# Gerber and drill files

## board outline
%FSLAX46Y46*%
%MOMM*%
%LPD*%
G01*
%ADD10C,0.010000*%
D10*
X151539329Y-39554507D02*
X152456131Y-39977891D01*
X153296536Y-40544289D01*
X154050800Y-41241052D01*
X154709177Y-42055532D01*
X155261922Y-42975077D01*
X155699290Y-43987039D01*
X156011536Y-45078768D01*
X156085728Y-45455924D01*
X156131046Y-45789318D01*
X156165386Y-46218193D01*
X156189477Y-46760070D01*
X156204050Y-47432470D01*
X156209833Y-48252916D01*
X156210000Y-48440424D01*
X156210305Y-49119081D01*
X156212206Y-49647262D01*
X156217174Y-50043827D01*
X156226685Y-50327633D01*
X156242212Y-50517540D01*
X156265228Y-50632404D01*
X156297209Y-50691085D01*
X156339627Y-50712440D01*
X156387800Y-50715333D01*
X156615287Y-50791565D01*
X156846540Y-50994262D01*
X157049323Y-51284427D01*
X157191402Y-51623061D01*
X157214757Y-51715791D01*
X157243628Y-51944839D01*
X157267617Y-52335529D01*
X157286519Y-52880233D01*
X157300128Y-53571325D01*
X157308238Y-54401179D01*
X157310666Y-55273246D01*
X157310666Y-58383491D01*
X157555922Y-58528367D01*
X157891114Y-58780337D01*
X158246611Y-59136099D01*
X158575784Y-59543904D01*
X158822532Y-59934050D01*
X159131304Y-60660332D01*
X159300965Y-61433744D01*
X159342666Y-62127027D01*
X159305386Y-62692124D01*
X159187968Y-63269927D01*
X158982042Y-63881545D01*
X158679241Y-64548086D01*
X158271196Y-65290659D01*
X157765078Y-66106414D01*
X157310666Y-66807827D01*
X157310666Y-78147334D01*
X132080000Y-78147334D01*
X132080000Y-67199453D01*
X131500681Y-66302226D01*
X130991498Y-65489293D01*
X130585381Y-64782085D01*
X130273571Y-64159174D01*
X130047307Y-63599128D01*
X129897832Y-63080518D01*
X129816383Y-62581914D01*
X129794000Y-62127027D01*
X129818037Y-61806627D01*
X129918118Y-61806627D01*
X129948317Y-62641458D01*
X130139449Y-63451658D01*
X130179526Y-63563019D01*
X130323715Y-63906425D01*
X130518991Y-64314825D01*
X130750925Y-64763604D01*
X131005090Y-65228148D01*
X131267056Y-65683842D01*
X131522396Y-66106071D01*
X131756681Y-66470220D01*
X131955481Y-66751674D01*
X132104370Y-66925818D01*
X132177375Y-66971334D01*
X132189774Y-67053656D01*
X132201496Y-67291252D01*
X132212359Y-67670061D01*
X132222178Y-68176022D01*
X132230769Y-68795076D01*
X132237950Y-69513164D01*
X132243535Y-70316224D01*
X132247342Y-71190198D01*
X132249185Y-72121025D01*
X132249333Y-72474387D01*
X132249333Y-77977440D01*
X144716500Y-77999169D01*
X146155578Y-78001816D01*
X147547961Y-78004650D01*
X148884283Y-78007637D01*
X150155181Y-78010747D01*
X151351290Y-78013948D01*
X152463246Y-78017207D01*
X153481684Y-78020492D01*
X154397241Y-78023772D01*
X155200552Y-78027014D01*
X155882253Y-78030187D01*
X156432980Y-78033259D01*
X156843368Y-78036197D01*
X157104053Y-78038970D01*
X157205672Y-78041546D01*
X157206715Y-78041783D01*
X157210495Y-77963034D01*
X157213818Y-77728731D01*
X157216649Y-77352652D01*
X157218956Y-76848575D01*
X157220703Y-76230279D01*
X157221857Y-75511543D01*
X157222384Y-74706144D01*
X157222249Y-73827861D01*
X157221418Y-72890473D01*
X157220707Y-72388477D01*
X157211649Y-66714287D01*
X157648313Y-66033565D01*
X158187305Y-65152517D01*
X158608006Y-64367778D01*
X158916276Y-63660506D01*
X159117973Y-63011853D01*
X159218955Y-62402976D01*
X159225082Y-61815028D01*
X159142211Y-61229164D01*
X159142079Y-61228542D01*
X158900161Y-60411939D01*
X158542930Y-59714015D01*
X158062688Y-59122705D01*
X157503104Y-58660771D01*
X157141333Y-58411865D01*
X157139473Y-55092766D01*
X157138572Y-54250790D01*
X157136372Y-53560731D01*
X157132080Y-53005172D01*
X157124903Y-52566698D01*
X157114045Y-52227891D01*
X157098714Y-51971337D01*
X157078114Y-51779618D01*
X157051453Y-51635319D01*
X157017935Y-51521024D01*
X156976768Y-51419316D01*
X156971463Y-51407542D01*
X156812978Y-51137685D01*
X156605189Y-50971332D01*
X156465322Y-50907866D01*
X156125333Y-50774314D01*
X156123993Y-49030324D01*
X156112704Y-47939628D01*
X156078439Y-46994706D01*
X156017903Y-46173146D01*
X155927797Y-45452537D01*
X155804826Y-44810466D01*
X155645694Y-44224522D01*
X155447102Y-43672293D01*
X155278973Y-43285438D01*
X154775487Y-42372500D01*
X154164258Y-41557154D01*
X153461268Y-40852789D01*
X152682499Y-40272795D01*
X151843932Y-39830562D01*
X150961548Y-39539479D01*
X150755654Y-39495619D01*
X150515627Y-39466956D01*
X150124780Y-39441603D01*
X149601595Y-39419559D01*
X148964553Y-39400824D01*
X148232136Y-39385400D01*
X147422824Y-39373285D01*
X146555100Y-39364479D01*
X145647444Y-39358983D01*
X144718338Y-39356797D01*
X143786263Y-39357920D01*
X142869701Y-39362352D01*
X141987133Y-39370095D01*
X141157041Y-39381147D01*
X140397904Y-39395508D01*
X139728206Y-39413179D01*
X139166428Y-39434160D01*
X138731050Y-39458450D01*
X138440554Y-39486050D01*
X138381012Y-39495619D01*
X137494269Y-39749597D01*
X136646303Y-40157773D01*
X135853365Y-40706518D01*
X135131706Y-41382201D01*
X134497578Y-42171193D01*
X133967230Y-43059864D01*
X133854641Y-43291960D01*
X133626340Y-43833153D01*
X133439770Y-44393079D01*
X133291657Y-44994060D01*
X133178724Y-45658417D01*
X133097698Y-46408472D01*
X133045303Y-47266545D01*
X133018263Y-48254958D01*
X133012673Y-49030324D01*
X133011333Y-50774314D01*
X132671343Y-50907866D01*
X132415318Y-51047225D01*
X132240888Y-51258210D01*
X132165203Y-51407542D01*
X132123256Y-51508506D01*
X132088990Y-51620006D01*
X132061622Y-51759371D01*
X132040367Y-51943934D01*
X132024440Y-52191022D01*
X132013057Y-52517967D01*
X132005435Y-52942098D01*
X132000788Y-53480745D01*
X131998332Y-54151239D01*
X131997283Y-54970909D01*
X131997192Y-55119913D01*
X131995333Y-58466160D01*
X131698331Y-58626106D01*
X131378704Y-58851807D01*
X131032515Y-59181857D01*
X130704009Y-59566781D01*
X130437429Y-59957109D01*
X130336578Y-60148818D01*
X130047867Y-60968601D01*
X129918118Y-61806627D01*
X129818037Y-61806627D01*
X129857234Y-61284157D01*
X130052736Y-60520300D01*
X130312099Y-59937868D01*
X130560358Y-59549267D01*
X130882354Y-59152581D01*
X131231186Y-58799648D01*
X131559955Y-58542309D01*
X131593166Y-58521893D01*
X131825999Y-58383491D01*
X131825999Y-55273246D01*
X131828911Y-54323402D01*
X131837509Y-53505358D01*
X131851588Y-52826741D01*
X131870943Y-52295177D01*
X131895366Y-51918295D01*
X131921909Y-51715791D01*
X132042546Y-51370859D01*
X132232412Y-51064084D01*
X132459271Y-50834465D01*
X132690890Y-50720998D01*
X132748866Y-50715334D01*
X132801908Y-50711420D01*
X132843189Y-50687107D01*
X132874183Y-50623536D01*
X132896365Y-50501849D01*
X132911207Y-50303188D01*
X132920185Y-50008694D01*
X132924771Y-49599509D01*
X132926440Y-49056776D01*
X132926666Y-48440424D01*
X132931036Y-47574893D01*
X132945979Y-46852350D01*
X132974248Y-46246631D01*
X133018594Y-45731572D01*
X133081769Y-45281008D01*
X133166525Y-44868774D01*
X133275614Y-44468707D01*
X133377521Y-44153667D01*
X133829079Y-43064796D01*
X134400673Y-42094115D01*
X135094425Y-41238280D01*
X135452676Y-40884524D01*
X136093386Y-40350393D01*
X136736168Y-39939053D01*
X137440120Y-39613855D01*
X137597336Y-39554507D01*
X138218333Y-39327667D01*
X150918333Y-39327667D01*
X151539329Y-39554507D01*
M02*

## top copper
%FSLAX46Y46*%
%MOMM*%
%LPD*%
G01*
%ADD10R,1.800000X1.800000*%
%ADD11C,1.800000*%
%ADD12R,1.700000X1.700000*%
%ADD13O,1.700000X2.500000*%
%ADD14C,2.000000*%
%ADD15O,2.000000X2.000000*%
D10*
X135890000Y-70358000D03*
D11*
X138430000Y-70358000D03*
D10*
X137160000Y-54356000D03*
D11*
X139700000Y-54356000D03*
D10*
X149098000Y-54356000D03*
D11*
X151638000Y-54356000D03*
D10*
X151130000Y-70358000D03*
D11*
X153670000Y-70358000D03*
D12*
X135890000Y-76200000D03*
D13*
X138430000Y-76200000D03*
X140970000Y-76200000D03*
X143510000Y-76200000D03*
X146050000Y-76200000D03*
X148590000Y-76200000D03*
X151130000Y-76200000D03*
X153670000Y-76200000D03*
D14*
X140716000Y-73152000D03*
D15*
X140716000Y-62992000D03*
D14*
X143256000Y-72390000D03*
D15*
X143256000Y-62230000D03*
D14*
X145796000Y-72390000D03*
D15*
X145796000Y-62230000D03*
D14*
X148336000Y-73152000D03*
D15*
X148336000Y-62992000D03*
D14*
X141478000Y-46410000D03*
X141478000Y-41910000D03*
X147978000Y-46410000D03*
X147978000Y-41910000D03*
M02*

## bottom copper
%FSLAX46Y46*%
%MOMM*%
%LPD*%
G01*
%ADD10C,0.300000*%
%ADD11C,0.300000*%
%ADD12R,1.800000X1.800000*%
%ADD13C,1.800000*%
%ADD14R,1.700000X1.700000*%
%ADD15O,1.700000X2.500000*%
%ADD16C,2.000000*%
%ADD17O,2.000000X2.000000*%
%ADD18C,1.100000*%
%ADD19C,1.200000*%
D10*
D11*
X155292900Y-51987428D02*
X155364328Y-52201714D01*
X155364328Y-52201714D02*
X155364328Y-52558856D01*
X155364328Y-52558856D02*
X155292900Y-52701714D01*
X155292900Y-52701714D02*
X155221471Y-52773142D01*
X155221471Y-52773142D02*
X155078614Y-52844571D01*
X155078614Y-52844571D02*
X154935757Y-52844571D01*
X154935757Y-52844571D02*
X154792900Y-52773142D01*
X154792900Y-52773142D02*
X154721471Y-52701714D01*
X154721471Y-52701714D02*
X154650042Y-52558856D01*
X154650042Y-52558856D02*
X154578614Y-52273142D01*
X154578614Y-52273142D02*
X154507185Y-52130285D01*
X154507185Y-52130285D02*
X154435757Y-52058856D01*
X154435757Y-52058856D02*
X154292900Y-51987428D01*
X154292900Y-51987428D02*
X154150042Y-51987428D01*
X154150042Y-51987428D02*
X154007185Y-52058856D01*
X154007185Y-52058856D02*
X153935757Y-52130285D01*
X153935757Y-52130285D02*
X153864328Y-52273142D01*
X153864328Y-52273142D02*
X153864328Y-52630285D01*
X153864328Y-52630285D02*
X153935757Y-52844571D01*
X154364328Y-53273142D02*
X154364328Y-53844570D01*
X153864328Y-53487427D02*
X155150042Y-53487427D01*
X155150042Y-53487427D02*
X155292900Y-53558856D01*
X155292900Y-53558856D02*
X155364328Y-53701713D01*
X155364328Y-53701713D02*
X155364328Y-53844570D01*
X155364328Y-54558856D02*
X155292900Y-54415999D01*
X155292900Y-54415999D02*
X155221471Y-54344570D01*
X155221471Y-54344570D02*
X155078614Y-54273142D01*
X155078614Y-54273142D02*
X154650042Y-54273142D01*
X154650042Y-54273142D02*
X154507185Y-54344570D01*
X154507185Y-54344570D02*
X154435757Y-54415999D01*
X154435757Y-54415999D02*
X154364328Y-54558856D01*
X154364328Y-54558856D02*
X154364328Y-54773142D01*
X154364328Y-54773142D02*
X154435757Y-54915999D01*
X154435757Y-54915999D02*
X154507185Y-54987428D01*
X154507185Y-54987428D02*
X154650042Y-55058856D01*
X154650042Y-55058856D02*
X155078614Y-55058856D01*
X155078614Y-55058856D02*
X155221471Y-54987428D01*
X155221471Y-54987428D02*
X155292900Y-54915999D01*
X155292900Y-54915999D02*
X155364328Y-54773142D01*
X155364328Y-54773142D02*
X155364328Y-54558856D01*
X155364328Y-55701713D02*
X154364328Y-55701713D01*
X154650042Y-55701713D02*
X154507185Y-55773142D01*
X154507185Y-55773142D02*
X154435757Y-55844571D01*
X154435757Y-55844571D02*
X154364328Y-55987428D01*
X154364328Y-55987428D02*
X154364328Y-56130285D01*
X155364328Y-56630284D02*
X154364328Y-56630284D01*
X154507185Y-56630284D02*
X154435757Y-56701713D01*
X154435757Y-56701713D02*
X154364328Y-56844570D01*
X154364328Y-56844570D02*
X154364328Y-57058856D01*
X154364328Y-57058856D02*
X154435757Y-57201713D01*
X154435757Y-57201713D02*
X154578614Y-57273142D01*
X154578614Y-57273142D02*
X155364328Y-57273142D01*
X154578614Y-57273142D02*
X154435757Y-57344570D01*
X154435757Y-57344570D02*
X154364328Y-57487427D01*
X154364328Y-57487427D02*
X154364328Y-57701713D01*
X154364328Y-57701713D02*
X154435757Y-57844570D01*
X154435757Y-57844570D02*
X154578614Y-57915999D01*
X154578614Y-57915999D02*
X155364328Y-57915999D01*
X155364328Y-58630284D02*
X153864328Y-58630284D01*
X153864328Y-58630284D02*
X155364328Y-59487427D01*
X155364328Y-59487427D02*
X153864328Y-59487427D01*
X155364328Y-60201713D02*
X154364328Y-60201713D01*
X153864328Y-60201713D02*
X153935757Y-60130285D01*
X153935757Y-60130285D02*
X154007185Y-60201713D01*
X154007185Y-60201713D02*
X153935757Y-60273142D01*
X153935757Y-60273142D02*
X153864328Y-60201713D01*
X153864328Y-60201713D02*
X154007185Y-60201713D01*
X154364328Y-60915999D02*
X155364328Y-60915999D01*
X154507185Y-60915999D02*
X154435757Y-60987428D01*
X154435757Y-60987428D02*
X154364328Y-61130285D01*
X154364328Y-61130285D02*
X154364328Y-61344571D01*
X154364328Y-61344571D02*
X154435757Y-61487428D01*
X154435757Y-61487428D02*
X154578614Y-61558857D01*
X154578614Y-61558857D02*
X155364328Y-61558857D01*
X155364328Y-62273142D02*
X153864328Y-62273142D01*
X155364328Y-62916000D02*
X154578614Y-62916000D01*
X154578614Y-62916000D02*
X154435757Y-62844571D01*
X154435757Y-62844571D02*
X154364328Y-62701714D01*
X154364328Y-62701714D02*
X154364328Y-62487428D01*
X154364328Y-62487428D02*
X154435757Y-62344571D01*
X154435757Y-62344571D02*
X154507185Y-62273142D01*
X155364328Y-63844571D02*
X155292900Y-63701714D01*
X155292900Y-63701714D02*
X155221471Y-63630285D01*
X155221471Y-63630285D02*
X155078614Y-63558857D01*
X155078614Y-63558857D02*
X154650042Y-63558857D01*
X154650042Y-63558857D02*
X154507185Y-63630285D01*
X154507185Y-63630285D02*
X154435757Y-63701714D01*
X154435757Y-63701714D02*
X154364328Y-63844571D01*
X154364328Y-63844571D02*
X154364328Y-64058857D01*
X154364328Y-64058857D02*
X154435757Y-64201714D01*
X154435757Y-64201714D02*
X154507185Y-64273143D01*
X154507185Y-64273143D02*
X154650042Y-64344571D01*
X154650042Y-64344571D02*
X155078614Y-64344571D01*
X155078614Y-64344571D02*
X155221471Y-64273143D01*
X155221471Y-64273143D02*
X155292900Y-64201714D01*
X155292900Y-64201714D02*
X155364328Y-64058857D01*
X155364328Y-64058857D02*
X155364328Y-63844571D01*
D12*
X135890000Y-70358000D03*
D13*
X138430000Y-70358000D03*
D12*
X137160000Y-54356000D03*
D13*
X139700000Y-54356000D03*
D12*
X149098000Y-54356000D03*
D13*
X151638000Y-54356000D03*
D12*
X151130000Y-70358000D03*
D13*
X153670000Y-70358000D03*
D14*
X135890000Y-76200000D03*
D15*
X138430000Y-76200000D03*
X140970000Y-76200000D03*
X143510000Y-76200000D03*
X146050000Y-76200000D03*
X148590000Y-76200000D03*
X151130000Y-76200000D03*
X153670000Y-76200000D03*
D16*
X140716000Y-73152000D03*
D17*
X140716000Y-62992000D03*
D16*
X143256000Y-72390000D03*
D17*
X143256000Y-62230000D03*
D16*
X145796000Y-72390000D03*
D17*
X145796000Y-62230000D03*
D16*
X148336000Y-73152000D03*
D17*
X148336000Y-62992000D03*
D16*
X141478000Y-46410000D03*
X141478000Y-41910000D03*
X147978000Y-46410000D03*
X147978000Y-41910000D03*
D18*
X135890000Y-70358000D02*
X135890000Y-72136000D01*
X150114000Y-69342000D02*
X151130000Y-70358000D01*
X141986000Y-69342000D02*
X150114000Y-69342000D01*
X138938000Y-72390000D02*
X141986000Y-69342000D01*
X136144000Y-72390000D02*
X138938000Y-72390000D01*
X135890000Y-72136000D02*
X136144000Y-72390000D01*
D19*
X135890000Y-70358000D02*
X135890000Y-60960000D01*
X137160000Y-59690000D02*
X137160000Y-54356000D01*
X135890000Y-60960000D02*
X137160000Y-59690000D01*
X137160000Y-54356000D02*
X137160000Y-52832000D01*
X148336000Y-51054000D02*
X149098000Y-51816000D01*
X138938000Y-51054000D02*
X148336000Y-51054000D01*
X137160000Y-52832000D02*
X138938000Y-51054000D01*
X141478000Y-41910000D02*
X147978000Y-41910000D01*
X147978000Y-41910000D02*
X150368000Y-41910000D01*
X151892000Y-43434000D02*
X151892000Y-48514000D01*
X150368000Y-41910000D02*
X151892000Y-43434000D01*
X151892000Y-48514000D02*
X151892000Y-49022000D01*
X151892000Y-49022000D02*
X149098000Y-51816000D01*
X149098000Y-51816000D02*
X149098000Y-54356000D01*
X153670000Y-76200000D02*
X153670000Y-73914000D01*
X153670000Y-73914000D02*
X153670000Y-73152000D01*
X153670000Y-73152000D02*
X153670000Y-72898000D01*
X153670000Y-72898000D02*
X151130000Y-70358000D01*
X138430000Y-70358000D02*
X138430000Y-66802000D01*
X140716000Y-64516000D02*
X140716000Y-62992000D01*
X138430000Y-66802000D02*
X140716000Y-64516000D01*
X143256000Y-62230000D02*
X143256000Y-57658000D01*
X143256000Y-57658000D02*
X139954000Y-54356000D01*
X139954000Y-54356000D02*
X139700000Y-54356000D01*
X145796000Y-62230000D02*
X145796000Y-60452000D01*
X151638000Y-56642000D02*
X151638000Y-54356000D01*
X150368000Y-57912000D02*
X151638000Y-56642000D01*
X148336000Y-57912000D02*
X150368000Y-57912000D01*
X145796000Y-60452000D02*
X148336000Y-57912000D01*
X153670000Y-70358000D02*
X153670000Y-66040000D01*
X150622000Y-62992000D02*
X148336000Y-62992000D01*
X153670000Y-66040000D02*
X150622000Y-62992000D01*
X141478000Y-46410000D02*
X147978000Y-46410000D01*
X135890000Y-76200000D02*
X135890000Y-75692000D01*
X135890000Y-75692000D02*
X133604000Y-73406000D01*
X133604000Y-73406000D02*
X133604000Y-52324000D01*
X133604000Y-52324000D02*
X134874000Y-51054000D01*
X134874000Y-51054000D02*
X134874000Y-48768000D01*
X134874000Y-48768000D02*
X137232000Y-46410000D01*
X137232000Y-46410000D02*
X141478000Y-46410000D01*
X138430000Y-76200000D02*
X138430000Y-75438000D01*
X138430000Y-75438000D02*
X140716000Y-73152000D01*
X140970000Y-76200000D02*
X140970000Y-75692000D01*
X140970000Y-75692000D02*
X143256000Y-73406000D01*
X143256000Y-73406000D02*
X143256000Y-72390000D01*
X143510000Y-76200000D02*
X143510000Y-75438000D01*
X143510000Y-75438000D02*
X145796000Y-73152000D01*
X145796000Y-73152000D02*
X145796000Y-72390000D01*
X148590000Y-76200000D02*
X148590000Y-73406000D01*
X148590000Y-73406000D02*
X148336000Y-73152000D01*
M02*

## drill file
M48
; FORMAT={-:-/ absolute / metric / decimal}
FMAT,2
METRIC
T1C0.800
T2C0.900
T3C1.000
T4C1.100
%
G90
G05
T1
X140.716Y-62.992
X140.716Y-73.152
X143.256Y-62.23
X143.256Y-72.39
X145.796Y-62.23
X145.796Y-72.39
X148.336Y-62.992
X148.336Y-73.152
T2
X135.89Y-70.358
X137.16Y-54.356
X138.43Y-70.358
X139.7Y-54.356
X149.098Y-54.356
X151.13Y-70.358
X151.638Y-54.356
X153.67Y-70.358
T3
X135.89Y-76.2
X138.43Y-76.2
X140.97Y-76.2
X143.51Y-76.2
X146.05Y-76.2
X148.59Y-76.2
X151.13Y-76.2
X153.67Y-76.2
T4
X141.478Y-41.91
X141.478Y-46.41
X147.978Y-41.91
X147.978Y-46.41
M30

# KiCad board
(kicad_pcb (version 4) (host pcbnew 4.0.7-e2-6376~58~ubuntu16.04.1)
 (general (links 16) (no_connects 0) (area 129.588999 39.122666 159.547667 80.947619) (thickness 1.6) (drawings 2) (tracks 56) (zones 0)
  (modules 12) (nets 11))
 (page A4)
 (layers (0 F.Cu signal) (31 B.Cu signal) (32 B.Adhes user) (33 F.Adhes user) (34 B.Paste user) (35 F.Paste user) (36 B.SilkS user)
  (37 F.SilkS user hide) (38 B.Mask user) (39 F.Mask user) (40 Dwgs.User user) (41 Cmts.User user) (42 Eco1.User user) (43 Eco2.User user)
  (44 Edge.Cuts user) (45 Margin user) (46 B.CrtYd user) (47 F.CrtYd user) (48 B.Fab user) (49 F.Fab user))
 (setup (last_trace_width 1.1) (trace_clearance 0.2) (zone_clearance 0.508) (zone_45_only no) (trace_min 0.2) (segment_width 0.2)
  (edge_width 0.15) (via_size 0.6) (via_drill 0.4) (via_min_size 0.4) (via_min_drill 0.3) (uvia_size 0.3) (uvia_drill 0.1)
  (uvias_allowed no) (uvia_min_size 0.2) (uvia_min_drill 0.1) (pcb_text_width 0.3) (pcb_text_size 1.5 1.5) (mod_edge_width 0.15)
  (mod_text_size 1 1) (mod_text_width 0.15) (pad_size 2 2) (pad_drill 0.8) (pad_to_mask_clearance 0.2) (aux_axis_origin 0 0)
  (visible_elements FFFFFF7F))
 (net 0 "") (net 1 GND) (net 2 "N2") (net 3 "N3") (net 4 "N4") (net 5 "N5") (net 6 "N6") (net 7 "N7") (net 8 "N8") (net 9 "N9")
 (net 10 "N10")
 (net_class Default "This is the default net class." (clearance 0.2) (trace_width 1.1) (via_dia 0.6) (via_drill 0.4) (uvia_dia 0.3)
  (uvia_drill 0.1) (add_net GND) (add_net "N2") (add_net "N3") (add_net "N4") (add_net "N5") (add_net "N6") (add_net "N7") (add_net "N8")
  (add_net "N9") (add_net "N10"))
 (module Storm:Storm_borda (layer F.Cu) (at 144.526 58.674)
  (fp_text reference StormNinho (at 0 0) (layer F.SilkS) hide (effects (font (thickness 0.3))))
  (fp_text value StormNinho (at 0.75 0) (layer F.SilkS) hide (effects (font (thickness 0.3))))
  (fp_poly
   (pts (xy 7.013329 -19.119493) (xy 7.930131 -18.696109) (xy 8.770536 -18.129711) (xy 9.5248 -17.432948) (xy 10.183177 -16.618468)
    (xy 10.735922 -15.698923) (xy 11.17329 -14.686961) (xy 11.485536 -13.595232) (xy 11.559728 -13.218076) (xy 11.605046 -12.884682)
    (xy 11.639386 -12.455807) (xy 11.663477 -11.91393) (xy 11.67805 -11.24153) (xy 11.683833 -10.421084) (xy 11.684 -10.233576)
    (xy 11.684305 -9.554919) (xy 11.686206 -9.026738) (xy 11.691174 -8.630173) (xy 11.700685 -8.346367) (xy 11.716212 -8.15646)
    (xy 11.739228 -8.041596) (xy 11.771209 -7.982915) (xy 11.813627 -7.96156) (xy 11.8618 -7.958667) (xy 12.089287 -7.882435)
    (xy 12.32054 -7.679738) (xy 12.523323 -7.389573) (xy 12.665402 -7.050939) (xy 12.688757 -6.958209) (xy 12.717628 -6.729161)
    (xy 12.741617 -6.338471) (xy 12.760519 -5.793767) (xy 12.774128 -5.102675) (xy 12.782238 -4.272821) (xy 12.784666 -3.400754)
    (xy 12.784666 -0.290509) (xy 13.029922 -0.145633) (xy 13.365114 0.106337) (xy 13.720611 0.462099) (xy 14.049784 0.869904)
    (xy 14.296532 1.26005) (xy 14.605304 1.986332) (xy 14.774965 2.759744) (xy 14.816666 3.453027) (xy 14.779386 4.018124)
    (xy 14.661968 4.595927) (xy 14.456042 5.207545) (xy 14.153241 5.874086) (xy 13.745196 6.616659) (xy 13.239078 7.432414)
    (xy 12.784666 8.133827) (xy 12.784666 19.473334) (xy -12.446 19.473334) (xy -12.446 8.525453) (xy -13.025319 7.628226)
    (xy -13.534502 6.815293) (xy -13.940619 6.108085) (xy -14.252429 5.485174) (xy -14.478693 4.925128) (xy -14.628168 4.406518)
    (xy -14.709617 3.907914) (xy -14.732 3.453027) (xy -14.707963 3.132627) (xy -14.607882 3.132627) (xy -14.577683 3.967458)
    (xy -14.386551 4.777658) (xy -14.346474 4.889019) (xy -14.202285 5.232425) (xy -14.007009 5.640825) (xy -13.775075 6.089604)
    (xy -13.52091 6.554148) (xy -13.258944 7.009842) (xy -13.003604 7.432071) (xy -12.769319 7.79622) (xy -12.570519 8.077674)
    (xy -12.42163 8.251818) (xy -12.348625 8.297334) (xy -12.336226 8.379656) (xy -12.324504 8.617252) (xy -12.313641 8.996061)
    (xy -12.303822 9.502022) (xy -12.295231 10.121076) (xy -12.28805 10.839164) (xy -12.282465 11.642224) (xy -12.278658 12.516198)
    (xy -12.276815 13.447025) (xy -12.276667 13.800387) (xy -12.276667 19.30344) (xy 0.1905 19.325169) (xy 1.629578 19.327816)
    (xy 3.021961 19.33065) (xy 4.358283 19.333637) (xy 5.629181 19.336747) (xy 6.82529 19.339948) (xy 7.937246 19.343207)
    (xy 8.955684 19.346492) (xy 9.871241 19.349772) (xy 10.674552 19.353014) (xy 11.356253 19.356187) (xy 11.90698 19.359259)
    (xy 12.317368 19.362197) (xy 12.578053 19.36497) (xy 12.679672 19.367546) (xy 12.680715 19.367783) (xy 12.684495 19.289034)
    (xy 12.687818 19.054731) (xy 12.690649 18.678652) (xy 12.692956 18.174575) (xy 12.694703 17.556279) (xy 12.695857 16.837543)
    (xy 12.696384 16.032144) (xy 12.696249 15.153861) (xy 12.695418 14.216473) (xy 12.694707 13.714477) (xy 12.685649 8.040287)
    (xy 13.122313 7.359565) (xy 13.661305 6.478517) (xy 14.082006 5.693778) (xy 14.390276 4.986506) (xy 14.591973 4.337853)
    (xy 14.692955 3.728976) (xy 14.699082 3.141028) (xy 14.616211 2.555164) (xy 14.616079 2.554542) (xy 14.374161 1.737939)
    (xy 14.01693 1.040015) (xy 13.536688 0.448705) (xy 12.977104 -0.013229) (xy 12.615333 -0.262135) (xy 12.613473 -3.581234)
    (xy 12.612572 -4.42321) (xy 12.610372 -5.113269) (xy 12.60608 -5.668828) (xy 12.598903 -6.107302) (xy 12.588045 -6.446109)
    (xy 12.572714 -6.702663) (xy 12.552114 -6.894382) (xy 12.525453 -7.038681) (xy 12.491935 -7.152976) (xy 12.450768 -7.254684)
    (xy 12.445463 -7.266458) (xy 12.286978 -7.536315) (xy 12.079189 -7.702668) (xy 11.939322 -7.766134) (xy 11.599333 -7.899686)
    (xy 11.597993 -9.643676) (xy 11.586704 -10.734372) (xy 11.552439 -11.679294) (xy 11.491903 -12.500854) (xy 11.401797 -13.221463)
    (xy 11.278826 -13.863534) (xy 11.119694 -14.449478) (xy 10.921102 -15.001707) (xy 10.752973 -15.388562) (xy 10.249487 -16.3015)
    (xy 9.638258 -17.116846) (xy 8.935268 -17.821211) (xy 8.156499 -18.401205) (xy 7.317932 -18.843438) (xy 6.435548 -19.134521)
    (xy 6.229654 -19.178381) (xy 5.989627 -19.207044) (xy 5.59878 -19.232397) (xy 5.075595 -19.254441) (xy 4.438553 -19.273176)
    (xy 3.706136 -19.2886) (xy 2.896824 -19.300715) (xy 2.0291 -19.309521) (xy 1.121444 -19.315017) (xy 0.192338 -19.317203)
    (xy -0.739737 -19.31608) (xy -1.656299 -19.311648) (xy -2.538867 -19.303905) (xy -3.368959 -19.292853) (xy -4.128096 -19.278492)
    (xy -4.797794 -19.260821) (xy -5.359572 -19.23984) (xy -5.79495 -19.21555) (xy -6.085446 -19.18795) (xy -6.144988 -19.178381)
    (xy -7.031731 -18.924403) (xy -7.879697 -18.516227) (xy -8.672635 -17.967482) (xy -9.394294 -17.291799) (xy -10.028422 -16.502807)
    (xy -10.55877 -15.614136) (xy -10.671359 -15.38204) (xy -10.89966 -14.840847) (xy -11.08623 -14.280921) (xy -11.234343 -13.67994)
    (xy -11.347276 -13.015583) (xy -11.428302 -12.265528) (xy -11.480697 -11.407455) (xy -11.507737 -10.419042) (xy -11.513327 -9.643676)
    (xy -11.514667 -7.899686) (xy -11.854657 -7.766134) (xy -12.110682 -7.626775) (xy -12.285112 -7.41579) (xy -12.360797 -7.266458)
    (xy -12.402744 -7.165494) (xy -12.43701 -7.053994) (xy -12.464378 -6.914629) (xy -12.485633 -6.730066) (xy -12.50156 -6.482978)
    (xy -12.512943 -6.156033) (xy -12.520565 -5.731902) (xy -12.525212 -5.193255) (xy -12.527668 -4.522761) (xy -12.528717 -3.703091)
    (xy -12.528808 -3.554087) (xy -12.530667 -0.20784) (xy -12.827669 -0.047894) (xy -13.147296 0.177807) (xy -13.493485 0.507857)
    (xy -13.821991 0.892781) (xy -14.088571 1.283109) (xy -14.189422 1.474818) (xy -14.478133 2.294601) (xy -14.607882 3.132627)
    (xy -14.707963 3.132627) (xy -14.668766 2.610157) (xy -14.473264 1.8463) (xy -14.213901 1.263868) (xy -13.965642 0.875267)
    (xy -13.643646 0.478581) (xy -13.294814 0.125648) (xy -12.966045 -0.131691) (xy -12.932834 -0.152107) (xy -12.700001 -0.290509)
    (xy -12.700001 -3.400754) (xy -12.697089 -4.350598) (xy -12.688491 -5.168642) (xy -12.674412 -5.847259) (xy -12.655057 -6.378823)
    (xy -12.630634 -6.755705) (xy -12.604091 -6.958209) (xy -12.483454 -7.303141) (xy -12.293588 -7.609916) (xy -12.066729 -7.839535)
    (xy -11.83511 -7.953002) (xy -11.777134 -7.958666) (xy -11.724092 -7.96258) (xy -11.682811 -7.986893) (xy -11.651817 -8.050464)
    (xy -11.629635 -8.172151) (xy -11.614793 -8.370812) (xy -11.605815 -8.665306) (xy -11.601229 -9.074491) (xy -11.59956 -9.617224)
    (xy -11.599334 -10.233576) (xy -11.594964 -11.099107) (xy -11.580021 -11.82165) (xy -11.551752 -12.427369) (xy -11.507406 -12.942428)
    (xy -11.444231 -13.392992) (xy -11.359475 -13.805226) (xy -11.250386 -14.205293) (xy -11.148479 -14.520333) (xy -10.696921 -15.609204)
    (xy -10.125327 -16.579885) (xy -9.431575 -17.43572) (xy -9.073324 -17.789476) (xy -8.432614 -18.323607) (xy -7.789832 -18.734947)
    (xy -7.08588 -19.060145) (xy -6.928664 -19.119493) (xy -6.307667 -19.346333) (xy 6.392333 -19.346333) (xy 7.013329 -19.119493))
   (layer Edge.Cuts) (width 0.01)))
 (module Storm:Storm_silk (layer F.Cu) (at 144.526 57.404)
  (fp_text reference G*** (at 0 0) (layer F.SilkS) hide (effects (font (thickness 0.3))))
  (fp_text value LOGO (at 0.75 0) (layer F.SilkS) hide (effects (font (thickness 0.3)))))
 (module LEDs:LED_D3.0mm (layer F.Cu) (at 135.89 70.358)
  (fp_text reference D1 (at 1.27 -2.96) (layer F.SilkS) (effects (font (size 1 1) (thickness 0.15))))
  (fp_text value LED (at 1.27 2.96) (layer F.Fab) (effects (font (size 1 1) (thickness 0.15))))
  (pad 1 thru_hole rect (at 0 0) (size 1.8 1.8) (drill 0.9) (layers *.Cu *.Mask) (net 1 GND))
  (pad 2 thru_hole circle (at 2.54 0) (size 1.8 1.8) (drill 0.9) (layers *.Cu *.Mask) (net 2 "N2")))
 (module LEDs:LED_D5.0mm (layer F.Cu) (at 137.16 54.356)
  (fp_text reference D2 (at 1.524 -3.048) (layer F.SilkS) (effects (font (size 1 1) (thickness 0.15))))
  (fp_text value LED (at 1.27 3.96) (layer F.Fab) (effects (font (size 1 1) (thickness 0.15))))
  (pad 1 thru_hole rect (at 0 0) (size 1.8 1.8) (drill 0.9) (layers *.Cu *.Mask) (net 1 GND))
  (pad 2 thru_hole circle (at 2.54 0) (size 1.8 1.8) (drill 0.9) (layers *.Cu *.Mask) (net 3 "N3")))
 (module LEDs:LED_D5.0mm (layer F.Cu) (at 149.098 54.356)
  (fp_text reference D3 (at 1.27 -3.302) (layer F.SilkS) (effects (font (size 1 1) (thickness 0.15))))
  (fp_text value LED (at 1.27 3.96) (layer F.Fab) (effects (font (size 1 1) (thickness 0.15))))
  (pad 1 thru_hole rect (at 0 0) (size 1.8 1.8) (drill 0.9) (layers *.Cu *.Mask) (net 1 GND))
  (pad 2 thru_hole circle (at 2.54 0) (size 1.8 1.8) (drill 0.9) (layers *.Cu *.Mask) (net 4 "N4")))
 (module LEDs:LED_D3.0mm (layer F.Cu) (at 151.13 70.358)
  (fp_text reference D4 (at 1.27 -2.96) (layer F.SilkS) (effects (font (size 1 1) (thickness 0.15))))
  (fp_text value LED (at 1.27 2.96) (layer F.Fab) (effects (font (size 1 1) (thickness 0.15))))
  (pad 1 thru_hole rect (at 0 0) (size 1.8 1.8) (drill 0.9) (layers *.Cu *.Mask) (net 1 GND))
  (pad 2 thru_hole circle (at 2.54 0) (size 1.8 1.8) (drill 0.9) (layers *.Cu *.Mask) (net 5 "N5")))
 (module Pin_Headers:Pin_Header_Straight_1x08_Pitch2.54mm (layer F.Cu) (at 135.89 76.2 90)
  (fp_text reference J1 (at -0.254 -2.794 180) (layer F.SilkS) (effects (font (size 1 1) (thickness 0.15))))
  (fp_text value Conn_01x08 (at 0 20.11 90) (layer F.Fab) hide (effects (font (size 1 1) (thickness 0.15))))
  (pad 1 thru_hole rect (at 0 0 90) (size 1.7 1.7) (drill 1) (layers *.Cu *.Mask) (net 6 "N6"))
  (pad 2 thru_hole oval (at 0 2.54 90) (size 2.5 1.7) (drill 1) (layers *.Cu *.Mask) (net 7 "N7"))
  (pad 3 thru_hole oval (at 0 5.08 90) (size 2.5 1.7) (drill 1) (layers *.Cu *.Mask) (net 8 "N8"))
  (pad 4 thru_hole oval (at 0 7.62 90) (size 2.5 1.7) (drill 1) (layers *.Cu *.Mask) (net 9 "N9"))
  (pad 5 thru_hole oval (at 0 10.16 90) (size 2.5 1.7) (drill 1) (layers *.Cu *.Mask))
  (pad 6 thru_hole oval (at 0 12.7 90) (size 2.5 1.7) (drill 1) (layers *.Cu *.Mask) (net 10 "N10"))
  (pad 7 thru_hole oval (at 0 15.24 90) (size 2.5 1.7) (drill 1) (layers *.Cu *.Mask))
  (pad 8 thru_hole oval (at 0 17.78 90) (size 2.5 1.7) (drill 1) (layers *.Cu *.Mask) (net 1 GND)))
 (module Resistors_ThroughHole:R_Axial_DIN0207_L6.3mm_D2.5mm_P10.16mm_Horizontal (layer F.Cu) (at 140.716 73.152 90)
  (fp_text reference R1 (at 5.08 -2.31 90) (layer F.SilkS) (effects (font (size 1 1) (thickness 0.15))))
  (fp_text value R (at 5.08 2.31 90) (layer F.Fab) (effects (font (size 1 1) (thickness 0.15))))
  (pad 1 thru_hole circle (at 0 0 90) (size 2 2) (drill 0.8) (layers *.Cu *.Mask) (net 7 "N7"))
  (pad 2 thru_hole oval (at 10.16 0 90) (size 2 2) (drill 0.8) (layers *.Cu *.Mask) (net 2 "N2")))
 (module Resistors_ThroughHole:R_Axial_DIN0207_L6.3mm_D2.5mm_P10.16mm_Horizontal (layer F.Cu) (at 143.256 72.39 90)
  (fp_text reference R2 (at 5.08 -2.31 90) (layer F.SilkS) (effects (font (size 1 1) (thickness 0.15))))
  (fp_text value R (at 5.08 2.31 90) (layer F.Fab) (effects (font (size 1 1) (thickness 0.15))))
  (pad 1 thru_hole circle (at 0 0 90) (size 2 2) (drill 0.8) (layers *.Cu *.Mask) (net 8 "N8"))
  (pad 2 thru_hole oval (at 10.16 0 90) (size 2 2) (drill 0.8) (layers *.Cu *.Mask) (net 3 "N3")))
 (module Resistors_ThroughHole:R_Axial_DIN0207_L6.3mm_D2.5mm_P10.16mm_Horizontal (layer F.Cu) (at 145.796 72.39 90)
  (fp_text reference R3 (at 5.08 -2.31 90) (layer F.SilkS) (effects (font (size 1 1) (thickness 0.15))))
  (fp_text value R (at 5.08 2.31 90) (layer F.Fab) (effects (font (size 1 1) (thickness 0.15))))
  (pad 1 thru_hole circle (at 0 0 90) (size 2 2) (drill 0.8) (layers *.Cu *.Mask) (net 9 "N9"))
  (pad 2 thru_hole oval (at 10.16 0 90) (size 2 2) (drill 0.8) (layers *.Cu *.Mask) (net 4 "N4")))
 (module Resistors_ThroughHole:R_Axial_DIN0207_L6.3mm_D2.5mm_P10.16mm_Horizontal (layer F.Cu) (at 148.336 73.152 90)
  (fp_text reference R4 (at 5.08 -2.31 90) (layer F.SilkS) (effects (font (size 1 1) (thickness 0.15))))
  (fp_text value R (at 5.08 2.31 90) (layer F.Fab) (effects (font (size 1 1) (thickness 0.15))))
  (pad 1 thru_hole circle (at 0 0 90) (size 2 2) (drill 0.8) (layers *.Cu *.Mask) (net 10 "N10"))
  (pad 2 thru_hole oval (at 10.16 0 90) (size 2 2) (drill 0.8) (layers *.Cu *.Mask) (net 5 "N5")))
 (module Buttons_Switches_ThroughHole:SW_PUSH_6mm (layer F.Cu) (at 141.478 41.91)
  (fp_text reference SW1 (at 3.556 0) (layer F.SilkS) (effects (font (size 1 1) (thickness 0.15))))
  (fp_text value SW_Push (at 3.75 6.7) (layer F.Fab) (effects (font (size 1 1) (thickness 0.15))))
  (pad 2 thru_hole circle (at 0 4.5 90) (size 2 2) (drill 1.1) (layers *.Cu *.Mask) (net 6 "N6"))
  (pad 1 thru_hole circle (at 0 0 90) (size 2 2) (drill 1.1) (layers *.Cu *.Mask) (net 1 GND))
  (pad 2 thru_hole circle (at 6.5 4.5 90) (size 2 2) (drill 1.1) (layers *.Cu *.Mask) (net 6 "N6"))
  (pad 1 thru_hole circle (at 6.5 0 90) (size 2 2) (drill 1.1) (layers *.Cu *.Mask) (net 1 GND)))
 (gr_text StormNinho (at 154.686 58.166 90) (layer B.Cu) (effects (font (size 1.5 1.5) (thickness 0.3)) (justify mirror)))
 (segment (start 135.89 70.358) (end 135.89 72.136) (width 1.1) (layer B.Cu) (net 1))
 (segment (start 150.114 69.342) (end 151.13 70.358) (width 1.1) (layer B.Cu) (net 1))
 (segment (start 141.986 69.342) (end 150.114 69.342) (width 1.1) (layer B.Cu) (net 1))
 (segment (start 138.938 72.39) (end 141.986 69.342) (width 1.1) (layer B.Cu) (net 1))
 (segment (start 136.144 72.39) (end 138.938 72.39) (width 1.1) (layer B.Cu) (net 1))
 (segment (start 135.89 72.136) (end 136.144 72.39) (width 1.1) (layer B.Cu) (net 1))
 (segment (start 135.89 70.358) (end 135.89 60.96) (width 1.2) (layer B.Cu) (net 1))
 (segment (start 137.16 59.69) (end 137.16 54.356) (width 1.2) (layer B.Cu) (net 1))
 (segment (start 135.89 60.96) (end 137.16 59.69) (width 1.2) (layer B.Cu) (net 1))
 (segment (start 137.16 54.356) (end 137.16 52.832) (width 1.2) (layer B.Cu) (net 1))
 (segment (start 148.336 51.054) (end 149.098 51.816) (width 1.2) (layer B.Cu) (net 1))
 (segment (start 138.938 51.054) (end 148.336 51.054) (width 1.2) (layer B.Cu) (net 1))
 (segment (start 137.16 52.832) (end 138.938 51.054) (width 1.2) (layer B.Cu) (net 1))
 (segment (start 141.478 41.91) (end 147.978 41.91) (width 1.2) (layer B.Cu) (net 1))
 (segment (start 147.978 41.91) (end 150.368 41.91) (width 1.2) (layer B.Cu) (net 1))
 (segment (start 151.892 43.434) (end 151.892 48.514) (width 1.2) (layer B.Cu) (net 1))
 (segment (start 150.368 41.91) (end 151.892 43.434) (width 1.2) (layer B.Cu) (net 1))
 (segment (start 151.892 48.514) (end 151.892 49.022) (width 1.2) (layer B.Cu) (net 1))
 (segment (start 151.892 49.022) (end 149.098 51.816) (width 1.2) (layer B.Cu) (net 1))
 (segment (start 149.098 51.816) (end 149.098 54.356) (width 1.2) (layer B.Cu) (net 1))
 (segment (start 153.67 76.2) (end 153.67 73.914) (width 1.2) (layer B.Cu) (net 1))
 (segment (start 153.67 73.914) (end 153.67 73.152) (width 1.2) (layer B.Cu) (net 1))
 (segment (start 153.67 73.152) (end 153.67 72.898) (width 1.2) (layer B.Cu) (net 1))
 (segment (start 153.67 72.898) (end 151.13 70.358) (width 1.2) (layer B.Cu) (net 1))
 (segment (start 138.43 70.358) (end 138.43 66.802) (width 1.2) (layer B.Cu) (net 2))
 (segment (start 140.716 64.516) (end 140.716 62.992) (width 1.2) (layer B.Cu) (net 2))
 (segment (start 138.43 66.802) (end 140.716 64.516) (width 1.2) (layer B.Cu) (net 2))
 (segment (start 143.256 62.23) (end 143.256 57.658) (width 1.2) (layer B.Cu) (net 3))
 (segment (start 143.256 57.658) (end 139.954 54.356) (width 1.2) (layer B.Cu) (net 3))
 (segment (start 139.954 54.356) (end 139.7 54.356) (width 1.2) (layer B.Cu) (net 3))
 (segment (start 145.796 62.23) (end 145.796 60.452) (width 1.2) (layer B.Cu) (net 4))
 (segment (start 151.638 56.642) (end 151.638 54.356) (width 1.2) (layer B.Cu) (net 4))
 (segment (start 150.368 57.912) (end 151.638 56.642) (width 1.2) (layer B.Cu) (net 4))
 (segment (start 148.336 57.912) (end 150.368 57.912) (width 1.2) (layer B.Cu) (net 4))
 (segment (start 145.796 60.452) (end 148.336 57.912) (width 1.2) (layer B.Cu) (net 4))
 (segment (start 153.67 70.358) (end 153.67 66.04) (width 1.2) (layer B.Cu) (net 5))
 (segment (start 150.622 62.992) (end 148.336 62.992) (width 1.2) (layer B.Cu) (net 5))
 (segment (start 153.67 66.04) (end 150.622 62.992) (width 1.2) (layer B.Cu) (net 5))
 (segment (start 141.478 46.41) (end 147.978 46.41) (width 1.2) (layer B.Cu) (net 6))
 (segment (start 135.89 76.2) (end 135.89 75.692) (width 1.2) (layer B.Cu) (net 6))
 (segment (start 135.89 75.692) (end 133.604 73.406) (width 1.2) (layer B.Cu) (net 6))
 (segment (start 133.604 73.406) (end 133.604 52.324) (width 1.2) (layer B.Cu) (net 6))
 (segment (start 133.604 52.324) (end 134.874 51.054) (width 1.2) (layer B.Cu) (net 6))
 (segment (start 134.874 51.054) (end 134.874 48.768) (width 1.2) (layer B.Cu) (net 6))
 (segment (start 134.874 48.768) (end 137.232 46.41) (width 1.2) (layer B.Cu) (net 6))
 (segment (start 137.232 46.41) (end 141.478 46.41) (width 1.2) (layer B.Cu) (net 6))
 (segment (start 138.43 76.2) (end 138.43 75.438) (width 1.2) (layer B.Cu) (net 7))
 (segment (start 138.43 75.438) (end 140.716 73.152) (width 1.2) (layer B.Cu) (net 7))
 (segment (start 140.97 76.2) (end 140.97 75.692) (width 1.2) (layer B.Cu) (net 8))
 (segment (start 140.97 75.692) (end 143.256 73.406) (width 1.2) (layer B.Cu) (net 8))
 (segment (start 143.256 73.406) (end 143.256 72.39) (width 1.2) (layer B.Cu) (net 8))
 (segment (start 143.51 76.2) (end 143.51 75.438) (width 1.2) (layer B.Cu) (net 9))
 (segment (start 143.51 75.438) (end 145.796 73.152) (width 1.2) (layer B.Cu) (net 9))
 (segment (start 145.796 73.152) (end 145.796 72.39) (width 1.2) (layer B.Cu) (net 9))
 (segment (start 148.59 76.2) (end 148.59 73.406) (width 1.2) (layer B.Cu) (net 10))
 (segment (start 148.59 73.406) (end 148.336 73.152) (width 1.2) (layer B.Cu) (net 10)))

